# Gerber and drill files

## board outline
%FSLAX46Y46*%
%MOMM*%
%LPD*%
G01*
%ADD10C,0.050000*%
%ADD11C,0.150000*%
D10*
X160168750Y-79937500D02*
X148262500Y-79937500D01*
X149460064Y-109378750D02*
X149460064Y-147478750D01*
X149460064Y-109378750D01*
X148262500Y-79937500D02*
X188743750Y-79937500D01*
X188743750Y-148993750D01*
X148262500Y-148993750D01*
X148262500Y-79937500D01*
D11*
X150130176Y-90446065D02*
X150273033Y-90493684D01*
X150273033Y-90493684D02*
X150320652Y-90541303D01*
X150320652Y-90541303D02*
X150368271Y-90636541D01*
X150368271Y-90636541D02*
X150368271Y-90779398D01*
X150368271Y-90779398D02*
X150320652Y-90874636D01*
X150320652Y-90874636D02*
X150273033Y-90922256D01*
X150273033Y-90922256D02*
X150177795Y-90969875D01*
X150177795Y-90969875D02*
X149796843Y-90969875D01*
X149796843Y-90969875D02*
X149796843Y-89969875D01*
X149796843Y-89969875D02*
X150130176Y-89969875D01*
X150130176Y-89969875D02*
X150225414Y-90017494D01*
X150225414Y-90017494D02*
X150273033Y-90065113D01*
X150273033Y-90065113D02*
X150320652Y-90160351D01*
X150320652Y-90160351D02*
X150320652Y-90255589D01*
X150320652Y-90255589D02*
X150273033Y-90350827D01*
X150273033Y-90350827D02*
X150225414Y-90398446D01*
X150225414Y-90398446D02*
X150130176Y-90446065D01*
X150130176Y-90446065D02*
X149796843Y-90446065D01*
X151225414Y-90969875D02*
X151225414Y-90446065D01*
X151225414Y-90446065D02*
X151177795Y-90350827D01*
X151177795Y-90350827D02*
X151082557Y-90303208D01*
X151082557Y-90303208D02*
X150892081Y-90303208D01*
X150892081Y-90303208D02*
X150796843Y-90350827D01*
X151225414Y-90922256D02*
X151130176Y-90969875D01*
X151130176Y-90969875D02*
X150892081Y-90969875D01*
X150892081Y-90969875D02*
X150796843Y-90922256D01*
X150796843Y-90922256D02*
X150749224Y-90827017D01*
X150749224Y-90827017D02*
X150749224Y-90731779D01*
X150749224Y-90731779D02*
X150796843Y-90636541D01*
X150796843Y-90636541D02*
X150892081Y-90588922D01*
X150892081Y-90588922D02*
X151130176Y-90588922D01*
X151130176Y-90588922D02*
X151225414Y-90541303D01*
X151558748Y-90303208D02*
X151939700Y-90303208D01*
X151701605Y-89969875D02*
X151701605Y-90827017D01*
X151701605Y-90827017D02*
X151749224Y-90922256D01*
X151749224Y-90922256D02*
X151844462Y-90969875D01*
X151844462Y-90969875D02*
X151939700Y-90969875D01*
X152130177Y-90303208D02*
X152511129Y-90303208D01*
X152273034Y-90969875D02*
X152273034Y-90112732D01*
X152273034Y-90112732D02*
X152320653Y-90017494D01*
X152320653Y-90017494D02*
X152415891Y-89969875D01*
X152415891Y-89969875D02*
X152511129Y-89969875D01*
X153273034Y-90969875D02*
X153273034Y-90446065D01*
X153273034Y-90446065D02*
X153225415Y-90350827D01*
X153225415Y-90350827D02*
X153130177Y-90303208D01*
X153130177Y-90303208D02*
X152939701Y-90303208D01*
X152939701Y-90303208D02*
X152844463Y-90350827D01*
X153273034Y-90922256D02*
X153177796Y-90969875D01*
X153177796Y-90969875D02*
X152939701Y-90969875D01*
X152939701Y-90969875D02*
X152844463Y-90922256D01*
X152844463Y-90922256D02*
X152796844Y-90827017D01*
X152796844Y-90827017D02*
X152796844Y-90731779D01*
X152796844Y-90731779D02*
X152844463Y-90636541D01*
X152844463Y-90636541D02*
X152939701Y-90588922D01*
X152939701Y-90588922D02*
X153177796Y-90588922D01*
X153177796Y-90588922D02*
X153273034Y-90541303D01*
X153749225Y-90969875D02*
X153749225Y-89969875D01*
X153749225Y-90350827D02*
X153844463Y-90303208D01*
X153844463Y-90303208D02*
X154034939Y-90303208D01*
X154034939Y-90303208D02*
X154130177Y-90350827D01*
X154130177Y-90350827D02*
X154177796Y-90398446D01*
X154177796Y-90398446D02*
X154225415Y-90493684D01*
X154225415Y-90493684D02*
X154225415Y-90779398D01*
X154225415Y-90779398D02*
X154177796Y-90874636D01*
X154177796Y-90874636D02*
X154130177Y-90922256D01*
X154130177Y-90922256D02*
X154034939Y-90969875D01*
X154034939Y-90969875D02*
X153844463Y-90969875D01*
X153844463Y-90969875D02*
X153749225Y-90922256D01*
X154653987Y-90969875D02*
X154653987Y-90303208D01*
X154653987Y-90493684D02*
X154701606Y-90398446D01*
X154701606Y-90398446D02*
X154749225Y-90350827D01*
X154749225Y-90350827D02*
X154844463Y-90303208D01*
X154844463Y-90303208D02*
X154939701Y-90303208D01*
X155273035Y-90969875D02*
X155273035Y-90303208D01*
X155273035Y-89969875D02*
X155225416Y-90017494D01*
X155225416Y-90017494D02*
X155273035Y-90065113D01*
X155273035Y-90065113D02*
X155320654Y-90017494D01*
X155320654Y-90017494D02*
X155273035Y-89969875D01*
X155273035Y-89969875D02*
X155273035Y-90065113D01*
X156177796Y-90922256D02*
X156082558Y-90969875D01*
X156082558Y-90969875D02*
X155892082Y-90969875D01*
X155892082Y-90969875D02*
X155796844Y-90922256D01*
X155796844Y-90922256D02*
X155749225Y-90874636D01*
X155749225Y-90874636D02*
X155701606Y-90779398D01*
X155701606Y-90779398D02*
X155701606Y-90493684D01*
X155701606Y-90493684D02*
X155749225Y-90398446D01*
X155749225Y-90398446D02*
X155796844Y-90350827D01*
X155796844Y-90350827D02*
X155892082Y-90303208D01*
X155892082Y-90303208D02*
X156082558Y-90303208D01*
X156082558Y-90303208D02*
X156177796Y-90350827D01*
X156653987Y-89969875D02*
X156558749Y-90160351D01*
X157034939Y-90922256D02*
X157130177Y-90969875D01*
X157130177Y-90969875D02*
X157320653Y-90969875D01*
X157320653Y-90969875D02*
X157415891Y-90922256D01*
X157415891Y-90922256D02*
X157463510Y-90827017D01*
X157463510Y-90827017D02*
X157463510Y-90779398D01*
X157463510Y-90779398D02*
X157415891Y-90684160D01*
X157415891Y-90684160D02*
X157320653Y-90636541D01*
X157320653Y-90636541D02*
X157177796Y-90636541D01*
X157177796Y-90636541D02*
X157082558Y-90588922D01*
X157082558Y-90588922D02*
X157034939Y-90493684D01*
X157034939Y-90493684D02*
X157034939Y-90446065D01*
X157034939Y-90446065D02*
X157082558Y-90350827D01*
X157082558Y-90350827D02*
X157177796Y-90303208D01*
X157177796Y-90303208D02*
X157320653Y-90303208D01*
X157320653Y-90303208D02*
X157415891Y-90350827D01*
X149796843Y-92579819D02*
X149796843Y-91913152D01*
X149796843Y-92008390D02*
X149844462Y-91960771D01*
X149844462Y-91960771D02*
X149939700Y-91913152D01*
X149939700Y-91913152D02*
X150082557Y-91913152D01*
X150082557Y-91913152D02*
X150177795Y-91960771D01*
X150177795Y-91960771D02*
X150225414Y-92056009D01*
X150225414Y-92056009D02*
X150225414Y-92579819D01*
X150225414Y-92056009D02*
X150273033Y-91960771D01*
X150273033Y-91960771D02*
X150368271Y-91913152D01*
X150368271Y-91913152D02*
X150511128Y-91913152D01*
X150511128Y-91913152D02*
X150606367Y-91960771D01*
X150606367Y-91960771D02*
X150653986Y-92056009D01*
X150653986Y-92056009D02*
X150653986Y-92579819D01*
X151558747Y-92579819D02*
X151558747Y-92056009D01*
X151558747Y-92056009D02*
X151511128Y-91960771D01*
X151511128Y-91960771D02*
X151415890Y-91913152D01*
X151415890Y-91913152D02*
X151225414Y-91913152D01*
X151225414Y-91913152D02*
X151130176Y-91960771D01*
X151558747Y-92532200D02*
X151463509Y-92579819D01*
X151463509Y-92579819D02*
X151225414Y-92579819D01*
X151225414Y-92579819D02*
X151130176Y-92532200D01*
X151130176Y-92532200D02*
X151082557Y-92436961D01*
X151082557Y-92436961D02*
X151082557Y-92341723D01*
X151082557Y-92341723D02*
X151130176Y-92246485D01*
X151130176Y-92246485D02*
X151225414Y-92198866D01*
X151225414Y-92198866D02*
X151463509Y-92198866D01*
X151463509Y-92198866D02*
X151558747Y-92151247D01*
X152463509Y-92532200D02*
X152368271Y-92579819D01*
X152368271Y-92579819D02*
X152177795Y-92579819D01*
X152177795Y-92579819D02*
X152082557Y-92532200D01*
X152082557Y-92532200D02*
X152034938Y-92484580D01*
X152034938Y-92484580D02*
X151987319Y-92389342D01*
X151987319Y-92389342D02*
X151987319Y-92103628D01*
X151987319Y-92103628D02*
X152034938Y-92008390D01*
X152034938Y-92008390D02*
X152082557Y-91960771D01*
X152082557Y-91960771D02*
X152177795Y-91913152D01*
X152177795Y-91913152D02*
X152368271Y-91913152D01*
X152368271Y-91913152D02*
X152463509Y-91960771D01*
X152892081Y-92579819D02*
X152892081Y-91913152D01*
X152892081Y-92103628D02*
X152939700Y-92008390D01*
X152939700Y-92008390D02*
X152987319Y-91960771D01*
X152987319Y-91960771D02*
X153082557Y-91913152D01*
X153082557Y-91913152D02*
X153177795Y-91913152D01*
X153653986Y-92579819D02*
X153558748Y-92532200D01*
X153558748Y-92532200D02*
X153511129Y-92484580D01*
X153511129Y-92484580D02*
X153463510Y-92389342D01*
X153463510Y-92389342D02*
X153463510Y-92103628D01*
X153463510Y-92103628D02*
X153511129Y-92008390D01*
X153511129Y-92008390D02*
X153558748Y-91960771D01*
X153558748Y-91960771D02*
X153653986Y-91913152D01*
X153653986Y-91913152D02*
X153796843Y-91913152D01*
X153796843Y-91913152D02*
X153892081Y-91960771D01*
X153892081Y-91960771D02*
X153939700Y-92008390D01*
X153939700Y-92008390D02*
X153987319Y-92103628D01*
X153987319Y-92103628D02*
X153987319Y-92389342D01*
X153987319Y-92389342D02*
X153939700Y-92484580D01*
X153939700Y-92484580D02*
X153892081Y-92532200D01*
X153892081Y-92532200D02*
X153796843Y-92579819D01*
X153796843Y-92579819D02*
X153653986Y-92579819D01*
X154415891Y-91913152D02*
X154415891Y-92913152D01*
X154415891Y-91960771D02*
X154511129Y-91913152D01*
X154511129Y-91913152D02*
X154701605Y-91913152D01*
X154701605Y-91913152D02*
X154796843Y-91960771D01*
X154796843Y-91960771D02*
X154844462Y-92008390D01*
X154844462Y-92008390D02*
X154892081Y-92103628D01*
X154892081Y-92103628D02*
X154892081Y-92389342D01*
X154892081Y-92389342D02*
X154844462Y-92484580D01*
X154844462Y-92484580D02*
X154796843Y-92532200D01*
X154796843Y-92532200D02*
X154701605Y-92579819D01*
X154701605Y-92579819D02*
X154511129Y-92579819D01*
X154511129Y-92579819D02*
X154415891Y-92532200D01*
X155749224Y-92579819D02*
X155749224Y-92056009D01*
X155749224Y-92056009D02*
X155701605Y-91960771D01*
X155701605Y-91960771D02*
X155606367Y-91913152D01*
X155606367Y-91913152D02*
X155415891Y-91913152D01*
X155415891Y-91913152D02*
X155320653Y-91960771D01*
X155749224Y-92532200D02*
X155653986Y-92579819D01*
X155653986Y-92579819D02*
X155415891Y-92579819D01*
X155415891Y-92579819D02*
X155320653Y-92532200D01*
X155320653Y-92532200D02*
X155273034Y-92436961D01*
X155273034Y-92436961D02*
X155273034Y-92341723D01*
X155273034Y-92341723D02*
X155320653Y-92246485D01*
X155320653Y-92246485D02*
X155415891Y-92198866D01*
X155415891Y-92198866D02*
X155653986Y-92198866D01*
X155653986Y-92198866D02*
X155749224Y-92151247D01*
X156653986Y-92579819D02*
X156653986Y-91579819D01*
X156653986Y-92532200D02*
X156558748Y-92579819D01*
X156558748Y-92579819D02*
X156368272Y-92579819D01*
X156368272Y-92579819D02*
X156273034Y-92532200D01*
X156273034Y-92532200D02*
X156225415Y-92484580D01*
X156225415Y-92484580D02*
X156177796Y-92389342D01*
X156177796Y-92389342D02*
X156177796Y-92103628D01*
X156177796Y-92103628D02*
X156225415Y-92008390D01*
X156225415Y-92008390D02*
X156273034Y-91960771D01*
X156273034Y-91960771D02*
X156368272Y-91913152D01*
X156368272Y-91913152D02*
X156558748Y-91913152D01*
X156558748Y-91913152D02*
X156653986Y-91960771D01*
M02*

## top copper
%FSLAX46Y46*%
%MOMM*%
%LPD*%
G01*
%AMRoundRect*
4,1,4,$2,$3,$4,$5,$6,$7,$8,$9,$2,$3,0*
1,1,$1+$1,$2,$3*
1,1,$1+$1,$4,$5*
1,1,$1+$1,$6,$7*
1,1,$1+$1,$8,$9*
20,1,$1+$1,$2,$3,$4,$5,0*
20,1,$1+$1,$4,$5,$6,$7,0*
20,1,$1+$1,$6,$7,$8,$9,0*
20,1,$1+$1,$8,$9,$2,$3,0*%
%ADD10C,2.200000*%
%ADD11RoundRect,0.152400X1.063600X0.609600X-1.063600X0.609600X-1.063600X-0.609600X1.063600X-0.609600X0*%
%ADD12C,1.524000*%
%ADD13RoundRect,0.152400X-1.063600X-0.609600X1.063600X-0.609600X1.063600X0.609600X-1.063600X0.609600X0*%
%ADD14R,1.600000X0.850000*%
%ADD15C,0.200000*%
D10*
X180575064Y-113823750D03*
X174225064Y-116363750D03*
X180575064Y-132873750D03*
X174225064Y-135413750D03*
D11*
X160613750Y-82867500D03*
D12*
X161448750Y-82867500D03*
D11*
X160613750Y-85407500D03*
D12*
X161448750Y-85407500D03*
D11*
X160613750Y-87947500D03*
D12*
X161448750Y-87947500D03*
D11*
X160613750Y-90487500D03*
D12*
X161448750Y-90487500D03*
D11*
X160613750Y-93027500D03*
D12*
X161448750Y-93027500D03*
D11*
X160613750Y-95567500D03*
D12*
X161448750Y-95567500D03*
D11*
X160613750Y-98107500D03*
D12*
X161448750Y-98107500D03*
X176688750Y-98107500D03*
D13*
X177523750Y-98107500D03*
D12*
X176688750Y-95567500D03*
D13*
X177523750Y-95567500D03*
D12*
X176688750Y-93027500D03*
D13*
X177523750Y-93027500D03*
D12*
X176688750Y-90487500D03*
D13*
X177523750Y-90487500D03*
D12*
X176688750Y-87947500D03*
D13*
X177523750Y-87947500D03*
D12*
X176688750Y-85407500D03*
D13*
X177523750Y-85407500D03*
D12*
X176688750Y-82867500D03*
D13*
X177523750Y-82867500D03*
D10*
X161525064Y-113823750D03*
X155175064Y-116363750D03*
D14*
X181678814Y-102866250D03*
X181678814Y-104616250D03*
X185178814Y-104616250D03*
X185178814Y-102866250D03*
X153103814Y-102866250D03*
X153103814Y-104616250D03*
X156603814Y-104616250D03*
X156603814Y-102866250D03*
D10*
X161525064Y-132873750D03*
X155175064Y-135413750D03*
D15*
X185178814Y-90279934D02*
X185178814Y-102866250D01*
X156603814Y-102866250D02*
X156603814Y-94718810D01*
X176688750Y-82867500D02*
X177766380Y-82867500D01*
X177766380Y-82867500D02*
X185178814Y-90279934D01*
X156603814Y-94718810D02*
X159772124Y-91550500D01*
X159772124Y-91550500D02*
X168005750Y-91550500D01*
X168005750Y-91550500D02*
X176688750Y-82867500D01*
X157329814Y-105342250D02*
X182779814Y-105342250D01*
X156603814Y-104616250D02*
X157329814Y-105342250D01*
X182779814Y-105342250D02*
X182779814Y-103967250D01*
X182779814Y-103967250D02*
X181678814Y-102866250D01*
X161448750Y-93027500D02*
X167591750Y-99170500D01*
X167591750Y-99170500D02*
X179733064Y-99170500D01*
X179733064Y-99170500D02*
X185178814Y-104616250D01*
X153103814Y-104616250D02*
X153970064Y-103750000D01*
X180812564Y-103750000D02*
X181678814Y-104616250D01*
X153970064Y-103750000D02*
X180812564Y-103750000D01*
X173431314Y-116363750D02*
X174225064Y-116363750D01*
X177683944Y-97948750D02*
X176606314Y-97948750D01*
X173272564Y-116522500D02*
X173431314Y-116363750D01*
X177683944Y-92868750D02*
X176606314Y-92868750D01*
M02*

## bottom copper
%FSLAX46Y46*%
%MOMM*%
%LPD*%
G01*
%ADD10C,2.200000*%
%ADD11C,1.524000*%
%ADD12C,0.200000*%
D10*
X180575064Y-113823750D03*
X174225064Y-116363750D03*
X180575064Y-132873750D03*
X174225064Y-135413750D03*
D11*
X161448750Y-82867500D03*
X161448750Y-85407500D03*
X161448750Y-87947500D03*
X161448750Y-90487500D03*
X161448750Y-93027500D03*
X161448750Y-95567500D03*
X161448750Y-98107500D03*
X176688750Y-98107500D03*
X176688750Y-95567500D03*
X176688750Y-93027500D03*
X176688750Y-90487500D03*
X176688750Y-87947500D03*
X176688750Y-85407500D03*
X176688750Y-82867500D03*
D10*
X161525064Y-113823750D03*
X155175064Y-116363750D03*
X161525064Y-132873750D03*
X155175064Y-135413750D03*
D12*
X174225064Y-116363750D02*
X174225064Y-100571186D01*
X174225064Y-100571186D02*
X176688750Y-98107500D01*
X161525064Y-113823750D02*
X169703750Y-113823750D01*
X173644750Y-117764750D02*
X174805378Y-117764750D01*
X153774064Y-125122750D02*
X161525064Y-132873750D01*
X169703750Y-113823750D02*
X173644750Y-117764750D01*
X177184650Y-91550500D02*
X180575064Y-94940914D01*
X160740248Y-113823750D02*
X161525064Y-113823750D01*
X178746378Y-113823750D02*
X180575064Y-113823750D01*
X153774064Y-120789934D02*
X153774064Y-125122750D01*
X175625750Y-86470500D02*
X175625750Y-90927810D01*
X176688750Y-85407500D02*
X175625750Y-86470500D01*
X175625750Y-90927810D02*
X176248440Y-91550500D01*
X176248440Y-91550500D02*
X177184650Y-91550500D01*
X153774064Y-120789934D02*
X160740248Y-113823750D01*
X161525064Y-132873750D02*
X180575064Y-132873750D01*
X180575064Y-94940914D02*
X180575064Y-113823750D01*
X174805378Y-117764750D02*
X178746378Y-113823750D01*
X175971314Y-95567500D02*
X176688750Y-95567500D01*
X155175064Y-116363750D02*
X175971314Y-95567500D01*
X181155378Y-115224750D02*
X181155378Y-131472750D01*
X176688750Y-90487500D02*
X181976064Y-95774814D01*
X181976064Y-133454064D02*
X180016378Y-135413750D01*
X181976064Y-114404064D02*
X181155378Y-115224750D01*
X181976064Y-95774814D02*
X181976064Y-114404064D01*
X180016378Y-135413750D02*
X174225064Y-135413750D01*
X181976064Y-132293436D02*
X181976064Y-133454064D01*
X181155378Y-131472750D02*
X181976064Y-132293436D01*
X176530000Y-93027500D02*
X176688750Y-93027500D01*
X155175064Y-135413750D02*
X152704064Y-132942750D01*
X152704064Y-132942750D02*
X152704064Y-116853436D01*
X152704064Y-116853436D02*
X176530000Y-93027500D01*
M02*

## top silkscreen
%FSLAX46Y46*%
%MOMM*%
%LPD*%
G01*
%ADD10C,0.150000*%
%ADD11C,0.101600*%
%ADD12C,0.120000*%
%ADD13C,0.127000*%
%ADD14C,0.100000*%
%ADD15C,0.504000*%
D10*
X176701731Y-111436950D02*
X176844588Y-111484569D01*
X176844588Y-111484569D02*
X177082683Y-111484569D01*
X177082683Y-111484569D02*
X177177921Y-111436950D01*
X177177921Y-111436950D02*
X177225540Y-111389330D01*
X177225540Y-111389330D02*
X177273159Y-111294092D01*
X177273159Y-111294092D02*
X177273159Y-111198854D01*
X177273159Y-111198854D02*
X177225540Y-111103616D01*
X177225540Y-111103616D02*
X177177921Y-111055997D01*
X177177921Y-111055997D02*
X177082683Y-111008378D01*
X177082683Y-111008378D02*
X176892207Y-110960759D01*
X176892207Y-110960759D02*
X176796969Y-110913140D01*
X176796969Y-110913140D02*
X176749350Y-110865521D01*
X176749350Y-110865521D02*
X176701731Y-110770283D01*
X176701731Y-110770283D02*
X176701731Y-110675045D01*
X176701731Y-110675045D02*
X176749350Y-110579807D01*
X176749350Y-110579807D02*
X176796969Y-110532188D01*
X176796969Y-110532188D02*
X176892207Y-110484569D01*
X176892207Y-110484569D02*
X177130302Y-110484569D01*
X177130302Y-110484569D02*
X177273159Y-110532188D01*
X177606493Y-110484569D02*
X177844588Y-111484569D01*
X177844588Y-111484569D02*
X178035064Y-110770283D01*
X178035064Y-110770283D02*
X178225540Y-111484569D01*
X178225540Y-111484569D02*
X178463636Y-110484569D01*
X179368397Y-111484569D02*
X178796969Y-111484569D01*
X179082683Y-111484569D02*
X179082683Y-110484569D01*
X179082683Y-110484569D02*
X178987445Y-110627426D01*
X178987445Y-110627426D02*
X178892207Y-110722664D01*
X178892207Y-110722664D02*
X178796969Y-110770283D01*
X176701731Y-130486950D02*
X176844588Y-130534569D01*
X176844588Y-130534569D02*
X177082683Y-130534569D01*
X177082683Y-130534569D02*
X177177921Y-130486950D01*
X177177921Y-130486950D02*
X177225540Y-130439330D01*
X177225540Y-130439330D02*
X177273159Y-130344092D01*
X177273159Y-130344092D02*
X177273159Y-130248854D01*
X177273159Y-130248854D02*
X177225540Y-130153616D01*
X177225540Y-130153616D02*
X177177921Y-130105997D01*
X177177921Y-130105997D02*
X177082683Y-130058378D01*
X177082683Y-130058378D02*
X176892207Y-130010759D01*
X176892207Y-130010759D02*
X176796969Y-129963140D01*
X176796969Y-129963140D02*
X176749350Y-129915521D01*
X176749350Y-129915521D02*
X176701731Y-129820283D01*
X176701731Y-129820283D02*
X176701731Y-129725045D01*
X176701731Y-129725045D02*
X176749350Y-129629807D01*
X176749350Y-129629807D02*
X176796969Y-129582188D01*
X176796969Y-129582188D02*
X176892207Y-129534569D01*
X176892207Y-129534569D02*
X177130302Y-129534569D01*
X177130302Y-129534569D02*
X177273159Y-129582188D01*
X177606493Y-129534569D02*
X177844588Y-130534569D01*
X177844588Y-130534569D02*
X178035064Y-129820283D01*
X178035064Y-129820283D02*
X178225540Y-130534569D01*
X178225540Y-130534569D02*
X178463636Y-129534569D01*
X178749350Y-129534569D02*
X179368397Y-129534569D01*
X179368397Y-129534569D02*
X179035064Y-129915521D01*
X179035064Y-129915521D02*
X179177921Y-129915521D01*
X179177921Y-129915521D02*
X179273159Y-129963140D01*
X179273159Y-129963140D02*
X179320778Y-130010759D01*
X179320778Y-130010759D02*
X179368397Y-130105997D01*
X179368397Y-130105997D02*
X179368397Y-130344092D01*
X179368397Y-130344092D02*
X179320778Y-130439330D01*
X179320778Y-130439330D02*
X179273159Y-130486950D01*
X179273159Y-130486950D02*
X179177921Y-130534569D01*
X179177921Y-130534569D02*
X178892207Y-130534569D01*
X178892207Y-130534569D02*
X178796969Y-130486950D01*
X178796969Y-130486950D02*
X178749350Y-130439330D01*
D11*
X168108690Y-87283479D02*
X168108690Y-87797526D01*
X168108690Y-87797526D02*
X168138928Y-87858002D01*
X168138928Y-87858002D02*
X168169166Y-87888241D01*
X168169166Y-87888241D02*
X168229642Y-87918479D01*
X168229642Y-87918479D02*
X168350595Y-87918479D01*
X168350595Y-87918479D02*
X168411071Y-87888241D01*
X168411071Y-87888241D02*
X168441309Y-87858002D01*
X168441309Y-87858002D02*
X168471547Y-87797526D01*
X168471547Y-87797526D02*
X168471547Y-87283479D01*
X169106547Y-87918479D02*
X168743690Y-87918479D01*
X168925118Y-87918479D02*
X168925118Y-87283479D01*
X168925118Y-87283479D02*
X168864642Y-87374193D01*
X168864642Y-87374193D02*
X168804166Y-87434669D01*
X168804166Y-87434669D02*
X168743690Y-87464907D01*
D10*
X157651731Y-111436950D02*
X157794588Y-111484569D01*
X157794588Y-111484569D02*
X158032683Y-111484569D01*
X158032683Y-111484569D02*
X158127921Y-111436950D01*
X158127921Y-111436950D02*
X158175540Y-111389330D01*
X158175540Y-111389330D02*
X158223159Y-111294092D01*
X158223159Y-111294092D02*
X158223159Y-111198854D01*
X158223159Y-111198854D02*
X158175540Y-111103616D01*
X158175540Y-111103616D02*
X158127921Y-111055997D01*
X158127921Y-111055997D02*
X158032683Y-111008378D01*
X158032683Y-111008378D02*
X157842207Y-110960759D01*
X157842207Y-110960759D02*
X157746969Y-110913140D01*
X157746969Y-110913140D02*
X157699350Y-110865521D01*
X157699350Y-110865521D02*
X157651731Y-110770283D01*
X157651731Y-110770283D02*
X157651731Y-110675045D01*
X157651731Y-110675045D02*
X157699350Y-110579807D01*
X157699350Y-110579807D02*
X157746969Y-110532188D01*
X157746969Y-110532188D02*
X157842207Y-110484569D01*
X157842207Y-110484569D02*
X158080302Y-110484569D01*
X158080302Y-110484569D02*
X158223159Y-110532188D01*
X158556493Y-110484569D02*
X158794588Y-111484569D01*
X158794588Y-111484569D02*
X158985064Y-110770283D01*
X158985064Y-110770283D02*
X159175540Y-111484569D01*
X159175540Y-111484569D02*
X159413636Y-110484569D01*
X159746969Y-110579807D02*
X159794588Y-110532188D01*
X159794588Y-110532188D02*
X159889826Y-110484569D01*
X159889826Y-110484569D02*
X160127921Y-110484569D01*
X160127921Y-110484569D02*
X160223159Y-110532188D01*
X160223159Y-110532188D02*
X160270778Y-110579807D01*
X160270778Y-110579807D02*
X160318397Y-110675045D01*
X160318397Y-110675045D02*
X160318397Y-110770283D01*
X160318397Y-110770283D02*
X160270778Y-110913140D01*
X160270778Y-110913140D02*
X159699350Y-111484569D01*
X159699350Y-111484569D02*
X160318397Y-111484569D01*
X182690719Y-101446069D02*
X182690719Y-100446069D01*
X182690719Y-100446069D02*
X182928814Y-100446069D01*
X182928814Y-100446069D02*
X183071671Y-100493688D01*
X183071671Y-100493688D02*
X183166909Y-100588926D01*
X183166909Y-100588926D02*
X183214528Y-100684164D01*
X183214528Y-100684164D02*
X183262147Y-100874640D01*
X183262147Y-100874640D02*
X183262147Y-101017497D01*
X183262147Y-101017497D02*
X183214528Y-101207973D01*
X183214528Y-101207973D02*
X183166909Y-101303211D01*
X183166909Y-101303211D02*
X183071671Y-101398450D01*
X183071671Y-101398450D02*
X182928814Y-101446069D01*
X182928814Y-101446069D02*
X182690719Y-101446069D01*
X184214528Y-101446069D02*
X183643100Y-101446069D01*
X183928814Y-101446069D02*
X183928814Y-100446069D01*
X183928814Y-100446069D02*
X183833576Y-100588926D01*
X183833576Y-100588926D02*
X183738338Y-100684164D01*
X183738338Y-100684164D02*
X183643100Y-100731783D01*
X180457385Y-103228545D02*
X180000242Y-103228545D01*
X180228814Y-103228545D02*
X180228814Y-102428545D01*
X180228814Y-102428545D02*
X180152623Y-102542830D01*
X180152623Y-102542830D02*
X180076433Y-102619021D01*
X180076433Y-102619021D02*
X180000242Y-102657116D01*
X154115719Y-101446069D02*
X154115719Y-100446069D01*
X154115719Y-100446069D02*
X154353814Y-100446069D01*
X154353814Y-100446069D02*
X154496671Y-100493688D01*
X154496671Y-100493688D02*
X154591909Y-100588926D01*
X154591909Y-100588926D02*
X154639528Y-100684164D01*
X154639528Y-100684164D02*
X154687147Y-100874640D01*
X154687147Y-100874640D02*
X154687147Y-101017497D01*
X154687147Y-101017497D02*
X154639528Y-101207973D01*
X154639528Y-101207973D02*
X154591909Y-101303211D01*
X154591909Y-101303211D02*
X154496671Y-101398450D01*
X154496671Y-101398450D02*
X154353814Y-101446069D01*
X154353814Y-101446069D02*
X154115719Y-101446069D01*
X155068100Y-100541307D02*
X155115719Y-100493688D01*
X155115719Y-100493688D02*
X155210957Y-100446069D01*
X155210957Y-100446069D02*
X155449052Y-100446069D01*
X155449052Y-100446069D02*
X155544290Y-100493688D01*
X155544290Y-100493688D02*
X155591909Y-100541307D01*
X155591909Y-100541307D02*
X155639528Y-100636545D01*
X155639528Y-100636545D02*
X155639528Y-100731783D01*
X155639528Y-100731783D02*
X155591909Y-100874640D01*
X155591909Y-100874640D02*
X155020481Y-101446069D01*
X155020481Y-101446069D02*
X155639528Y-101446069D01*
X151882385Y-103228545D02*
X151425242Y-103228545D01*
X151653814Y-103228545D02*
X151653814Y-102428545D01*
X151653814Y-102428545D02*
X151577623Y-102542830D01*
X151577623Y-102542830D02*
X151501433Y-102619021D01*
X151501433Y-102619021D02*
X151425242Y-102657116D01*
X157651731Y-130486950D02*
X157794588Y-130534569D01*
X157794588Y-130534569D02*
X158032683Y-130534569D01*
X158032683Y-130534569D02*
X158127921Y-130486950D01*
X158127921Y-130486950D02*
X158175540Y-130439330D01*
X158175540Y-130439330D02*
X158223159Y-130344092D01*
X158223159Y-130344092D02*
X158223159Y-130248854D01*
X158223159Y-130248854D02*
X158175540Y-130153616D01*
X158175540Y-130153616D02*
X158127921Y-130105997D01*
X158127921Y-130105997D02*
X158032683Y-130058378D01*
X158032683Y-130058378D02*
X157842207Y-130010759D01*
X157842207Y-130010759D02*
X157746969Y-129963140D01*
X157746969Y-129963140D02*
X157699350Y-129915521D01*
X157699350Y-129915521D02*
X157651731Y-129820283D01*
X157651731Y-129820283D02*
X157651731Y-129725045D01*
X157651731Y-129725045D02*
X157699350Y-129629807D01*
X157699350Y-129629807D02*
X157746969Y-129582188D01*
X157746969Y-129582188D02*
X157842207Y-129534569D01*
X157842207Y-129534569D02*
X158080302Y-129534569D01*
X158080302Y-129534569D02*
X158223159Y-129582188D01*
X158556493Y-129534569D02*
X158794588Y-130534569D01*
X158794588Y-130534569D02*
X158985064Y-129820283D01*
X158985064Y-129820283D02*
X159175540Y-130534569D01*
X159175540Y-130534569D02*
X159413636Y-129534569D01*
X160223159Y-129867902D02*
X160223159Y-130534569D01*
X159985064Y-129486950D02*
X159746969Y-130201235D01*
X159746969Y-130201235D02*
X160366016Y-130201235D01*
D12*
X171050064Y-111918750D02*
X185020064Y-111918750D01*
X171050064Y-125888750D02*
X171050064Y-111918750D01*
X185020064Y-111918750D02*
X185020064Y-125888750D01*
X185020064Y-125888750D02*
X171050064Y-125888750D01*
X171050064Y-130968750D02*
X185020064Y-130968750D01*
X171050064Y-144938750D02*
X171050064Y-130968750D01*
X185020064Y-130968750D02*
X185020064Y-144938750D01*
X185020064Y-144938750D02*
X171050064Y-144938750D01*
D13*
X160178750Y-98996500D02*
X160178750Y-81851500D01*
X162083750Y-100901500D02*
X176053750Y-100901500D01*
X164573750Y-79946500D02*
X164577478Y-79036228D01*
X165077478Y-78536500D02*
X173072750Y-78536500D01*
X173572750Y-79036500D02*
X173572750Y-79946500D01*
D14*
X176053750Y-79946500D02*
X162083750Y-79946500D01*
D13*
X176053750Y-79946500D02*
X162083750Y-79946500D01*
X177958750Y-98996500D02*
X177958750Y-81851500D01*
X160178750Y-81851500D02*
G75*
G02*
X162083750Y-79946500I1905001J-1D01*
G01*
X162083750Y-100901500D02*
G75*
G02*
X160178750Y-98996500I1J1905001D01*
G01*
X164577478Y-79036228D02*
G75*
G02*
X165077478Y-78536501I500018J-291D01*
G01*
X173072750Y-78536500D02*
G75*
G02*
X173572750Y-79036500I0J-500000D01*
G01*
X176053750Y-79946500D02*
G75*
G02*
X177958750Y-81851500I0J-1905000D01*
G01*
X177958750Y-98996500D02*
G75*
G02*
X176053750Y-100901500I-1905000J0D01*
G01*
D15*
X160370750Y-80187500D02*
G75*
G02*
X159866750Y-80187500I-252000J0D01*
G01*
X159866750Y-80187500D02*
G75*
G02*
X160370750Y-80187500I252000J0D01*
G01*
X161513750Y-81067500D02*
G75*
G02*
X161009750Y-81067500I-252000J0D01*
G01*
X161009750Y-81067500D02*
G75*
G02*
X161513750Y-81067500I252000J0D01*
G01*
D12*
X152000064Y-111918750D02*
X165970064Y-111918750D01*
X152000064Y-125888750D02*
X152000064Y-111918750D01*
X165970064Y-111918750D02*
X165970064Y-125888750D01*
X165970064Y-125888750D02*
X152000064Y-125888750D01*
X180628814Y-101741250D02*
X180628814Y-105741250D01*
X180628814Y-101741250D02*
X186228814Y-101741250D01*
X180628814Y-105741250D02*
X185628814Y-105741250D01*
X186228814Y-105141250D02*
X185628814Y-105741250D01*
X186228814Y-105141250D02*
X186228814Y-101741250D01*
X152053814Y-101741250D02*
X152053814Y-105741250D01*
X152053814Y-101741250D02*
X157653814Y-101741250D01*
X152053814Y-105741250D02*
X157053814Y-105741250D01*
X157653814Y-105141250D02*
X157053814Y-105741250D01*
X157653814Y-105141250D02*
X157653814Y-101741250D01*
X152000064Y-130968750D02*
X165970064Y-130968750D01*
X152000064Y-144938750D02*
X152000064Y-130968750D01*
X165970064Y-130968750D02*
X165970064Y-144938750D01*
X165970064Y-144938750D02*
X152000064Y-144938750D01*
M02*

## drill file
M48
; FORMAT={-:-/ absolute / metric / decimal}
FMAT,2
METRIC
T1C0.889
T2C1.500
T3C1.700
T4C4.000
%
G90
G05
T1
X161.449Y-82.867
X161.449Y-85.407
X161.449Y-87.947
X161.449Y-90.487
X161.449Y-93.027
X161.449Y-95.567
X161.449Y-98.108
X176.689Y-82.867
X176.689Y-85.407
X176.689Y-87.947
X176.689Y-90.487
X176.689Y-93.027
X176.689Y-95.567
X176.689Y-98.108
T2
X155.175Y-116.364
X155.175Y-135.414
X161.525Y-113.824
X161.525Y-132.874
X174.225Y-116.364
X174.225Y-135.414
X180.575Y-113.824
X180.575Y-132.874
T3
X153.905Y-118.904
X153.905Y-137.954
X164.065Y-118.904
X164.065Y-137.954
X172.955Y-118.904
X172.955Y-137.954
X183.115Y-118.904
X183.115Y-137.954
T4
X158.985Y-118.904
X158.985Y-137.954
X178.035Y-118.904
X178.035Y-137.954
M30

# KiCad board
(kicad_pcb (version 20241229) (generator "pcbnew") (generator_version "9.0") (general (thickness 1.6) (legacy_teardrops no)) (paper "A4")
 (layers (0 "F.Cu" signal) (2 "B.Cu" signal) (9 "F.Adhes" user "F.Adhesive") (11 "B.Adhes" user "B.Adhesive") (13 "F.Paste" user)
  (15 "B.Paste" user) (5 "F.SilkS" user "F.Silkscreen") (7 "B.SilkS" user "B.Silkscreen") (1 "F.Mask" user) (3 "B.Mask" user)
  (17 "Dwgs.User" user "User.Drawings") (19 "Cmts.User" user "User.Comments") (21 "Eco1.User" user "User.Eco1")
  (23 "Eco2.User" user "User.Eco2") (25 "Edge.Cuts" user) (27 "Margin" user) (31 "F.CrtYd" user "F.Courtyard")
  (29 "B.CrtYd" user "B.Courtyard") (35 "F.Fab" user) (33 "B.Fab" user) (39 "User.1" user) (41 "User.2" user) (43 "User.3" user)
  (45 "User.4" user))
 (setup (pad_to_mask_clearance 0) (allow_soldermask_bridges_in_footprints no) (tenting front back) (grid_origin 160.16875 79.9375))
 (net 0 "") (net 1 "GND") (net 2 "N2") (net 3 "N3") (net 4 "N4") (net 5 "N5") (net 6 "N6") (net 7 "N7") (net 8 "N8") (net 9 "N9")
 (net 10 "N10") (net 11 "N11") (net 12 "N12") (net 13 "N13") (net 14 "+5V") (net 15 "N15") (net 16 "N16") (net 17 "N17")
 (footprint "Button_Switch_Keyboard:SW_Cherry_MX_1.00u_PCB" (layer "F.Cu") (at 180.575064 113.82375)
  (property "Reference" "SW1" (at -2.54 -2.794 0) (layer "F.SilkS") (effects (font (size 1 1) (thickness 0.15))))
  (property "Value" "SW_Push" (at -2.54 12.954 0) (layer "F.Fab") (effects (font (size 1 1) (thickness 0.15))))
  (fp_line (start -9.525 -1.905) (end 4.445 -1.905) (stroke (width 0.12) (type solid)) (layer "F.SilkS"))
  (fp_line (start -9.525 12.065) (end -9.525 -1.905) (stroke (width 0.12) (type solid)) (layer "F.SilkS"))
  (fp_line (start 4.445 -1.905) (end 4.445 12.065) (stroke (width 0.12) (type solid)) (layer "F.SilkS"))
  (fp_line (start 4.445 12.065) (end -9.525 12.065) (stroke (width 0.12) (type solid)) (layer "F.SilkS"))
  (pad "" np_thru_hole circle (at -7.62 5.08) (size 1.7 1.7) (drill 1.7) (layers "*.Cu" "*.Mask"))
  (pad "" np_thru_hole circle (at -2.54 5.08) (size 4 4) (drill 4) (layers "*.Cu" "*.Mask"))
  (pad "" np_thru_hole circle (at 2.54 5.08) (size 1.7 1.7) (drill 1.7) (layers "*.Cu" "*.Mask"))
  (pad "1" thru_hole circle (at 0 0) (size 2.2 2.2) (drill 1.5) (layers "*.Cu" "*.Mask") (remove_unused_layers no) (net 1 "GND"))
  (pad "2" thru_hole circle (at -6.35 2.54) (size 2.2 2.2) (drill 1.5) (layers "*.Cu" "*.Mask") (remove_unused_layers no) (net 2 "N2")))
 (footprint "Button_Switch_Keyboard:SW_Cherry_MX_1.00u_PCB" (layer "F.Cu") (at 180.575064 132.87375)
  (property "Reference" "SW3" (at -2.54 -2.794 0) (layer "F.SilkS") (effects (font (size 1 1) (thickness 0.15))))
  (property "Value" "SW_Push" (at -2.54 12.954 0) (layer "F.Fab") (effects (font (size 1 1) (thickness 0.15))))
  (fp_line (start -9.525 -1.905) (end 4.445 -1.905) (stroke (width 0.12) (type solid)) (layer "F.SilkS"))
  (fp_line (start -9.525 12.065) (end -9.525 -1.905) (stroke (width 0.12) (type solid)) (layer "F.SilkS"))
  (fp_line (start 4.445 -1.905) (end 4.445 12.065) (stroke (width 0.12) (type solid)) (layer "F.SilkS"))
  (fp_line (start 4.445 12.065) (end -9.525 12.065) (stroke (width 0.12) (type solid)) (layer "F.SilkS"))
  (pad "" np_thru_hole circle (at -7.62 5.08) (size 1.7 1.7) (drill 1.7) (layers "*.Cu" "*.Mask"))
  (pad "" np_thru_hole circle (at -2.54 5.08) (size 4 4) (drill 4) (layers "*.Cu" "*.Mask"))
  (pad "" np_thru_hole circle (at 2.54 5.08) (size 1.7 1.7) (drill 1.7) (layers "*.Cu" "*.Mask"))
  (pad "1" thru_hole circle (at 0 0) (size 2.2 2.2) (drill 1.5) (layers "*.Cu" "*.Mask") (remove_unused_layers no) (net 1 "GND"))
  (pad "2" thru_hole circle (at -6.35 2.54) (size 2.2 2.2) (drill 1.5) (layers "*.Cu" "*.Mask") (remove_unused_layers no) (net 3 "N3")))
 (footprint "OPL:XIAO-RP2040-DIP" (layer "F.Cu") (at 169.06875 90.4875)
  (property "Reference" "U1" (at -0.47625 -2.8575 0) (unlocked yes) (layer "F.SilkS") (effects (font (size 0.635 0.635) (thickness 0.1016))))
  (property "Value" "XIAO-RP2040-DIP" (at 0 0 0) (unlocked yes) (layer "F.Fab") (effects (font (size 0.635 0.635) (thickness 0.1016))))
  (fp_line (start -8.89 8.509) (end -8.89 -8.636) (stroke (width 0.127) (type solid)) (layer "F.SilkS"))
  (fp_line (start -6.985 10.414) (end 6.985 10.414) (stroke (width 0.127) (type solid)) (layer "F.SilkS"))
  (fp_line (start -4.495 -10.541) (end -4.491272 -11.451272) (stroke (width 0.127) (type solid)) (layer "F.SilkS"))
  (fp_line (start -3.991272 -11.951) (end 4.004 -11.951) (stroke (width 0.127) (type solid)) (layer "F.SilkS"))
  (fp_line (start 4.504 -11.451) (end 4.504 -10.541) (stroke (width 0.127) (type solid)) (layer "F.SilkS"))
  (fp_line (start 6.985 -10.541) (end -6.985 -10.541) (stroke (width 0.1) (type solid)) (layer "F.SilkS"))
  (fp_line (start 6.985 -10.541) (end -6.985 -10.541) (stroke (width 0.127) (type solid)) (layer "F.SilkS"))
  (fp_line (start 8.89 8.509) (end 8.89 -8.636) (stroke (width 0.127) (type solid)) (layer "F.SilkS"))
  (fp_arc (start -8.89 -8.636) (mid -8.332038 -9.983038) (end -6.985 -10.541) (stroke (width 0.127) (type solid)) (layer "F.SilkS"))
  (fp_arc (start -6.985 10.414) (mid -8.332038 9.856038) (end -8.89 8.509) (stroke (width 0.127) (type solid)) (layer "F.SilkS"))
  (fp_arc (start -4.491272 -11.451272) (mid -4.344728 -11.80464) (end -3.991272 -11.951) (stroke (width 0.127) (type default))
   (layer "F.SilkS"))
  (fp_arc (start 4.004 -11.951) (mid 4.357553 -11.804553) (end 4.504 -11.451) (stroke (width 0.127) (type default)) (layer "F.SilkS"))
  (fp_arc (start 6.985 -10.541) (mid 8.332038 -9.983038) (end 8.89 -8.636) (stroke (width 0.127) (type solid)) (layer "F.SilkS"))
  (fp_arc (start 8.89 8.509) (mid 8.332038 9.856038) (end 6.985 10.414) (stroke (width 0.127) (type solid)) (layer "F.SilkS"))
  (fp_circle (center -8.95 -10.3) (end -8.95 -10.554) (stroke (width 0.5) (type solid)) (fill yes) (layer "F.SilkS"))
  (fp_circle (center -7.807 -9.42) (end -7.807 -9.674) (stroke (width 0.5) (type solid)) (fill yes) (layer "F.SilkS"))
  (pad "1" smd roundrect (at -8.455 -7.62 180) (size 2.432 1.524) (layers "F.Cu" "F.Mask") (roundrect_rratio 0.1) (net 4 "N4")
   (thermal_bridge_angle 45))
  (pad "1" thru_hole circle (at -7.62 -7.62 180) (size 1.524 1.524) (drill 0.889) (layers "*.Cu" "*.Mask") (remove_unused_layers no)
   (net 4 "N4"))
  (pad "2" smd roundrect (at -8.455 -5.08 180) (size 2.432 1.524) (layers "F.Cu" "F.Mask") (roundrect_rratio 0.1) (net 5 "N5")
   (thermal_bridge_angle 45))
  (pad "2" thru_hole circle (at -7.62 -5.08 180) (size 1.524 1.524) (drill 0.889) (layers "*.Cu" "*.Mask") (remove_unused_layers no)
   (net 5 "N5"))
  (pad "3" smd roundrect (at -8.455 -2.54 180) (size 2.432 1.524) (layers "F.Cu" "F.Mask") (roundrect_rratio 0.1) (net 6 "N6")
   (thermal_bridge_angle 45))
  (pad "3" thru_hole circle (at -7.62 -2.54 180) (size 1.524 1.524) (drill 0.889) (layers "*.Cu" "*.Mask") (remove_unused_layers no)
   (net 6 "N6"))
  (pad "4" smd roundrect (at -8.455 0 180) (size 2.432 1.524) (layers "F.Cu" "F.Mask") (roundrect_rratio 0.1) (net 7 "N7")
   (thermal_bridge_angle 45))
  (pad "4" thru_hole circle (at -7.62 0 180) (size 1.524 1.524) (drill 0.889) (layers "*.Cu" "*.Mask") (remove_unused_layers no)
   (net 7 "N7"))
  (pad "5" smd roundrect (at -8.455 2.54 180) (size 2.432 1.524) (layers "F.Cu" "F.Mask") (roundrect_rratio 0.1) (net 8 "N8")
   (thermal_bridge_angle 45))
  (pad "5" thru_hole circle (at -7.62 2.54 180) (size 1.524 1.524) (drill 0.889) (layers "*.Cu" "*.Mask") (remove_unused_layers no)
   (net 8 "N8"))
  (pad "6" smd roundrect (at -8.455 5.08 180) (size 2.432 1.524) (layers "F.Cu" "F.Mask") (roundrect_rratio 0.1) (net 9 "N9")
   (thermal_bridge_angle 45))
  (pad "6" thru_hole circle (at -7.62 5.08 180) (size 1.524 1.524) (drill 0.889) (layers "*.Cu" "*.Mask") (remove_unused_layers no)
   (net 9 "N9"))
  (pad "7" smd roundrect (at -8.455 7.62 180) (size 2.432 1.524) (layers "F.Cu" "F.Mask") (roundrect_rratio 0.1) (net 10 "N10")
   (thermal_bridge_angle 45))
  (pad "7" thru_hole circle (at -7.62 7.62 180) (size 1.524 1.524) (drill 0.889) (layers "*.Cu" "*.Mask") (remove_unused_layers no)
   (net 10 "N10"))
  (pad "8" thru_hole circle (at 7.62 7.62) (size 1.524 1.524) (drill 0.889) (layers "*.Cu" "*.Mask") (remove_unused_layers no) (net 2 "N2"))
  (pad "8" smd roundrect (at 8.455 7.62) (size 2.432 1.524) (layers "F.Cu" "F.Mask") (roundrect_rratio 0.1) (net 2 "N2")
   (thermal_bridge_angle 45))
  (pad "9" thru_hole circle (at 7.62 5.08) (size 1.524 1.524) (drill 0.889) (layers "*.Cu" "*.Mask") (remove_unused_layers no)
   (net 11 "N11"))
  (pad "9" smd roundrect (at 8.455 5.08) (size 2.432 1.524) (layers "F.Cu" "F.Mask") (roundrect_rratio 0.1) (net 11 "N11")
   (thermal_bridge_angle 45))
  (pad "10" thru_hole circle (at 7.62 2.54) (size 1.524 1.524) (drill 0.889) (layers "*.Cu" "*.Mask") (remove_unused_layers no)
   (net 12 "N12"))
  (pad "10" smd roundrect (at 8.455 2.54) (size 2.432 1.524) (layers "F.Cu" "F.Mask") (roundrect_rratio 0.1) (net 12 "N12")
   (thermal_bridge_angle 45))
  (pad "11" thru_hole circle (at 7.62 0) (size 1.524 1.524) (drill 0.889) (layers "*.Cu" "*.Mask") (remove_unused_layers no) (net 3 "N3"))
  (pad "11" smd roundrect (at 8.455 0) (size 2.432 1.524) (layers "F.Cu" "F.Mask") (roundrect_rratio 0.1) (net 3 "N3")
   (thermal_bridge_angle 45))
  (pad "12" thru_hole circle (at 7.62 -2.54) (size 1.524 1.524) (drill 0.889) (layers "*.Cu" "*.Mask") (remove_unused_layers no)
   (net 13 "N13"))
  (pad "12" smd roundrect (at 8.455 -2.54) (size 2.432 1.524) (layers "F.Cu" "F.Mask") (roundrect_rratio 0.1) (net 13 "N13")
   (thermal_bridge_angle 45))
  (pad "13" thru_hole circle (at 7.62 -5.08) (size 1.524 1.524) (drill 0.889) (layers "*.Cu" "*.Mask") (remove_unused_layers no)
   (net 1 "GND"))
  (pad "13" smd roundrect (at 8.455 -5.08) (size 2.432 1.524) (layers "F.Cu" "F.Mask") (roundrect_rratio 0.1) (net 1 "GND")
   (thermal_bridge_angle 45))
  (pad "14" thru_hole circle (at 7.62 -7.62) (size 1.524 1.524) (drill 0.889) (layers "*.Cu" "*.Mask") (remove_unused_layers no)
   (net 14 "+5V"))
  (pad "14" smd roundrect (at 8.455 -7.62) (size 2.432 1.524) (layers "F.Cu" "F.Mask") (roundrect_rratio 0.1) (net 14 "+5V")
   (thermal_bridge_angle 45)))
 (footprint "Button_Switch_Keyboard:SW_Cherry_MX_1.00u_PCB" (layer "F.Cu") (at 161.525064 113.82375)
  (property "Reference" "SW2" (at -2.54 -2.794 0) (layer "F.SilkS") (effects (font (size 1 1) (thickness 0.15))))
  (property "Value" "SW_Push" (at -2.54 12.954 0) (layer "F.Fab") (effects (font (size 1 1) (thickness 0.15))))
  (fp_line (start -9.525 -1.905) (end 4.445 -1.905) (stroke (width 0.12) (type solid)) (layer "F.SilkS"))
  (fp_line (start -9.525 12.065) (end -9.525 -1.905) (stroke (width 0.12) (type solid)) (layer "F.SilkS"))
  (fp_line (start 4.445 -1.905) (end 4.445 12.065) (stroke (width 0.12) (type solid)) (layer "F.SilkS"))
  (fp_line (start 4.445 12.065) (end -9.525 12.065) (stroke (width 0.12) (type solid)) (layer "F.SilkS"))
  (pad "" np_thru_hole circle (at -7.62 5.08) (size 1.7 1.7) (drill 1.7) (layers "*.Cu" "*.Mask"))
  (pad "" np_thru_hole circle (at -2.54 5.08) (size 4 4) (drill 4) (layers "*.Cu" "*.Mask"))
  (pad "" np_thru_hole circle (at 2.54 5.08) (size 1.7 1.7) (drill 1.7) (layers "*.Cu" "*.Mask"))
  (pad "1" thru_hole circle (at 0 0) (size 2.2 2.2) (drill 1.5) (layers "*.Cu" "*.Mask") (remove_unused_layers no) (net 1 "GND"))
  (pad "2" thru_hole circle (at -6.35 2.54) (size 2.2 2.2) (drill 1.5) (layers "*.Cu" "*.Mask") (remove_unused_layers no) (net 11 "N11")))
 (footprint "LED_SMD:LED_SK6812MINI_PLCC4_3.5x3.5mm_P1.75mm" (layer "F.Cu") (at 183.428814 103.74125)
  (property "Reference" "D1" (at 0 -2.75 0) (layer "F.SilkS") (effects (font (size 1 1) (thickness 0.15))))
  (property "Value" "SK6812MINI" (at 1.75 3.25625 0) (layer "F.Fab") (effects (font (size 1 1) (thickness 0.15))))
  (fp_line (start -2.8 -2) (end -2.8 2) (stroke (width 0.12) (type default)) (layer "F.SilkS"))
  (fp_line (start -2.8 -2) (end 2.8 -2) (stroke (width 0.12) (type solid)) (layer "F.SilkS"))
  (fp_line (start -2.8 2) (end 2.2 2) (stroke (width 0.12) (type solid)) (layer "F.SilkS"))
  (fp_line (start 2.8 1.4) (end 2.2 2) (stroke (width 0.12) (type default)) (layer "F.SilkS"))
  (fp_line (start 2.8 1.4) (end 2.8 -2) (stroke (width 0.12) (type solid)) (layer "F.SilkS"))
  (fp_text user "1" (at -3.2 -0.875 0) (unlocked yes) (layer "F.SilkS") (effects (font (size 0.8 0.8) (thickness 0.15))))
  (pad "1" smd rect (at -1.75 -0.875) (size 1.6 0.85) (layers "F.Cu" "F.Mask" "F.Paste") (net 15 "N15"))
  (pad "2" smd rect (at -1.75 0.875) (size 1.6 0.85) (layers "F.Cu" "F.Mask" "F.Paste") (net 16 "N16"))
  (pad "3" smd rect (at 1.75 0.875) (size 1.6 0.85) (layers "F.Cu" "F.Mask" "F.Paste") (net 8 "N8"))
  (pad "4" smd rect (at 1.75 -0.875) (size 1.6 0.85) (layers "F.Cu" "F.Mask" "F.Paste") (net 14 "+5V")))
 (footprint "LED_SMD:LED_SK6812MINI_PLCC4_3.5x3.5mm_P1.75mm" (layer "F.Cu") (at 154.853814 103.74125)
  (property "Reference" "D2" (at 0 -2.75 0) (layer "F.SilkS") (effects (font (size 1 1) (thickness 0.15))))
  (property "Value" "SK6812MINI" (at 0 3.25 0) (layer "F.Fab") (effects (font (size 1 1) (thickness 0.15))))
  (fp_line (start -2.8 -2) (end -2.8 2) (stroke (width 0.12) (type default)) (layer "F.SilkS"))
  (fp_line (start -2.8 -2) (end 2.8 -2) (stroke (width 0.12) (type solid)) (layer "F.SilkS"))
  (fp_line (start -2.8 2) (end 2.2 2) (stroke (width 0.12) (type solid)) (layer "F.SilkS"))
  (fp_line (start 2.8 1.4) (end 2.2 2) (stroke (width 0.12) (type default)) (layer "F.SilkS"))
  (fp_line (start 2.8 1.4) (end 2.8 -2) (stroke (width 0.12) (type solid)) (layer "F.SilkS"))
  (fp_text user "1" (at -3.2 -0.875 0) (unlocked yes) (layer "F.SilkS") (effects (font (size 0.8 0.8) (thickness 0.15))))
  (pad "1" smd rect (at -1.75 -0.875) (size 1.6 0.85) (layers "F.Cu" "F.Mask" "F.Paste") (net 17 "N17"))
  (pad "2" smd rect (at -1.75 0.875) (size 1.6 0.85) (layers "F.Cu" "F.Mask" "F.Paste") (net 16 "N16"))
  (pad "3" smd rect (at 1.75 0.875) (size 1.6 0.85) (layers "F.Cu" "F.Mask" "F.Paste") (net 15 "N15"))
  (pad "4" smd rect (at 1.75 -0.875) (size 1.6 0.85) (layers "F.Cu" "F.Mask" "F.Paste") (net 14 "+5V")))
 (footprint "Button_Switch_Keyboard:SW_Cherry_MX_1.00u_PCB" (layer "F.Cu") (at 161.525064 132.87375)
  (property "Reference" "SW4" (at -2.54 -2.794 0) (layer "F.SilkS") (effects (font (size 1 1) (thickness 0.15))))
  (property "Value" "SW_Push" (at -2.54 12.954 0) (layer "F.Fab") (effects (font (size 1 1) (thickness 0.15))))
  (fp_line (start -9.525 -1.905) (end 4.445 -1.905) (stroke (width 0.12) (type solid)) (layer "F.SilkS"))
  (fp_line (start -9.525 12.065) (end -9.525 -1.905) (stroke (width 0.12) (type solid)) (layer "F.SilkS"))
  (fp_line (start 4.445 -1.905) (end 4.445 12.065) (stroke (width 0.12) (type solid)) (layer "F.SilkS"))
  (fp_line (start 4.445 12.065) (end -9.525 12.065) (stroke (width 0.12) (type solid)) (layer "F.SilkS"))
  (pad "" np_thru_hole circle (at -7.62 5.08) (size 1.7 1.7) (drill 1.7) (layers "*.Cu" "*.Mask"))
  (pad "" np_thru_hole circle (at -2.54 5.08) (size 4 4) (drill 4) (layers "*.Cu" "*.Mask"))
  (pad "" np_thru_hole circle (at 2.54 5.08) (size 1.7 1.7) (drill 1.7) (layers "*.Cu" "*.Mask"))
  (pad "1" thru_hole circle (at 0 0) (size 2.2 2.2) (drill 1.5) (layers "*.Cu" "*.Mask") (remove_unused_layers no) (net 1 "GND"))
  (pad "2" thru_hole circle (at -6.35 2.54) (size 2.2 2.2) (drill 1.5) (layers "*.Cu" "*.Mask") (remove_unused_layers no) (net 12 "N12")))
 (gr_line (start 160.16875 79.9375) (end 148.2625 79.9375) (stroke (width 0.05) (type default)) (layer "Edge.Cuts"))
 (gr_rect (start 149.460064 109.37875) (end 149.460064 147.47875) (stroke (width 0.05) (type default)) (fill no) (layer "Edge.Cuts"))
 (gr_rect (start 148.2625 79.9375) (end 188.74375 148.99375) (stroke (width 0.05) (type default)) (fill no) (layer "Edge.Cuts"))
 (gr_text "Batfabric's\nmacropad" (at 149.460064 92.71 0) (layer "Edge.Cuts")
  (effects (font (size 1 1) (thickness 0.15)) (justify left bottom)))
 (segment (start 185.178814 90.279934) (end 185.178814 102.86625) (width 0.2) (layer "F.Cu") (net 14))
 (segment (start 156.603814 102.86625) (end 156.603814 94.71881) (width 0.2) (layer "F.Cu") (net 14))
 (segment (start 176.68875 82.8675) (end 177.76638 82.8675) (width 0.2) (layer "F.Cu") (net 14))
 (segment (start 177.76638 82.8675) (end 185.178814 90.279934) (width 0.2) (layer "F.Cu") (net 14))
 (segment (start 156.603814 94.71881) (end 159.772124 91.5505) (width 0.2) (layer "F.Cu") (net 14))
 (segment (start 159.772124 91.5505) (end 168.00575 91.5505) (width 0.2) (layer "F.Cu") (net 14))
 (segment (start 168.00575 91.5505) (end 176.68875 82.8675) (width 0.2) (layer "F.Cu") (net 14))
 (segment (start 157.329814 105.34225) (end 182.779814 105.34225) (width 0.2) (layer "F.Cu") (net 15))
 (segment (start 156.603814 104.61625) (end 157.329814 105.34225) (width 0.2) (layer "F.Cu") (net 15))
 (segment (start 182.779814 105.34225) (end 182.779814 103.96725) (width 0.2) (layer "F.Cu") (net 15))
 (segment (start 182.779814 103.96725) (end 181.678814 102.86625) (width 0.2) (layer "F.Cu") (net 15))
 (segment (start 161.44875 93.0275) (end 167.59175 99.1705) (width 0.2) (layer "F.Cu") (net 8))
 (segment (start 167.59175 99.1705) (end 179.733064 99.1705) (width 0.2) (layer "F.Cu") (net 8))
 (segment (start 179.733064 99.1705) (end 185.178814 104.61625) (width 0.2) (layer "F.Cu") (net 8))
 (segment (start 153.103814 104.61625) (end 153.970064 103.75) (width 0.2) (layer "F.Cu") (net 16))
 (segment (start 180.812564 103.75) (end 181.678814 104.61625) (width 0.2) (layer "F.Cu") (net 16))
 (segment (start 153.970064 103.75) (end 180.812564 103.75) (width 0.2) (layer "F.Cu") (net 16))
 (segment (start 173.431314 116.36375) (end 174.225064 116.36375) (width 0.2) (layer "F.Cu") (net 2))
 (segment (start 177.683944 97.94875) (end 176.606314 97.94875) (width 0.2) (layer "F.Cu") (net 2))
 (segment (start 173.272564 116.5225) (end 173.431314 116.36375) (width 0.2) (layer "F.Cu") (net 2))
 (segment (start 174.225064 116.36375) (end 174.225064 100.571186) (width 0.2) (layer "B.Cu") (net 2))
 (segment (start 174.225064 100.571186) (end 176.68875 98.1075) (width 0.2) (layer "B.Cu") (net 2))
 (segment (start 161.525064 113.82375) (end 169.70375 113.82375) (width 0.2) (layer "B.Cu") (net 1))
 (segment (start 173.64475 117.76475) (end 174.805378 117.76475) (width 0.2) (layer "B.Cu") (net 1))
 (segment (start 153.774064 125.12275) (end 161.525064 132.87375) (width 0.2) (layer "B.Cu") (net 1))
 (segment (start 169.70375 113.82375) (end 173.64475 117.76475) (width 0.2) (layer "B.Cu") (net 1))
 (segment (start 177.18465 91.5505) (end 180.575064 94.940914) (width 0.2) (layer "B.Cu") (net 1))
 (segment (start 160.740248 113.82375) (end 161.525064 113.82375) (width 0.2) (layer "B.Cu") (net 1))
 (segment (start 178.746378 113.82375) (end 180.575064 113.82375) (width 0.2) (layer "B.Cu") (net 1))
 (segment (start 153.774064 120.789934) (end 153.774064 125.12275) (width 0.2) (layer "B.Cu") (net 1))
 (segment (start 175.62575 86.4705) (end 175.62575 90.92781) (width 0.2) (layer "B.Cu") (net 1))
 (segment (start 176.68875 85.4075) (end 175.62575 86.4705) (width 0.2) (layer "B.Cu") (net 1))
 (segment (start 175.62575 90.92781) (end 176.24844 91.5505) (width 0.2) (layer "B.Cu") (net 1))
 (segment (start 176.24844 91.5505) (end 177.18465 91.5505) (width 0.2) (layer "B.Cu") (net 1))
 (segment (start 153.774064 120.789934) (end 160.740248 113.82375) (width 0.2) (layer "B.Cu") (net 1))
 (segment (start 161.525064 132.87375) (end 180.575064 132.87375) (width 0.2) (layer "B.Cu") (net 1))
 (segment (start 180.575064 94.940914) (end 180.575064 113.82375) (width 0.2) (layer "B.Cu") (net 1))
 (segment (start 174.805378 117.76475) (end 178.746378 113.82375) (width 0.2) (layer "B.Cu") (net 1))
 (segment (start 175.971314 95.5675) (end 176.68875 95.5675) (width 0.2) (layer "B.Cu") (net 11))
 (segment (start 155.175064 116.36375) (end 175.971314 95.5675) (width 0.2) (layer "B.Cu") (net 11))
 (segment (start 181.155378 115.22475) (end 181.155378 131.47275) (width 0.2) (layer "B.Cu") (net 3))
 (segment (start 176.68875 90.4875) (end 181.976064 95.774814) (width 0.2) (layer "B.Cu") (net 3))
 (segment (start 181.976064 133.454064) (end 180.016378 135.41375) (width 0.2) (layer "B.Cu") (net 3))
 (segment (start 181.976064 114.404064) (end 181.155378 115.22475) (width 0.2) (layer "B.Cu") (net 3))
 (segment (start 181.976064 95.774814) (end 181.976064 114.404064) (width 0.2) (layer "B.Cu") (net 3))
 (segment (start 180.016378 135.41375) (end 174.225064 135.41375) (width 0.2) (layer "B.Cu") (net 3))
 (segment (start 181.976064 132.293436) (end 181.976064 133.454064) (width 0.2) (layer "B.Cu") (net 3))
 (segment (start 181.155378 131.47275) (end 181.976064 132.293436) (width 0.2) (layer "B.Cu") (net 3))
 (segment (start 177.683944 92.86875) (end 176.606314 92.86875) (width 0.2) (layer "F.Cu") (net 12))
 (segment (start 176.53 93.0275) (end 176.68875 93.0275) (width 0.2) (layer "B.Cu") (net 12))
 (segment (start 155.175064 135.41375) (end 152.704064 132.94275) (width 0.2) (layer "B.Cu") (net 12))
 (segment (start 152.704064 132.94275) (end 152.704064 116.853436) (width 0.2) (layer "B.Cu") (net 12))
 (segment (start 152.704064 116.853436) (end 176.53 93.0275) (width 0.2) (layer "B.Cu") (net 12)))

